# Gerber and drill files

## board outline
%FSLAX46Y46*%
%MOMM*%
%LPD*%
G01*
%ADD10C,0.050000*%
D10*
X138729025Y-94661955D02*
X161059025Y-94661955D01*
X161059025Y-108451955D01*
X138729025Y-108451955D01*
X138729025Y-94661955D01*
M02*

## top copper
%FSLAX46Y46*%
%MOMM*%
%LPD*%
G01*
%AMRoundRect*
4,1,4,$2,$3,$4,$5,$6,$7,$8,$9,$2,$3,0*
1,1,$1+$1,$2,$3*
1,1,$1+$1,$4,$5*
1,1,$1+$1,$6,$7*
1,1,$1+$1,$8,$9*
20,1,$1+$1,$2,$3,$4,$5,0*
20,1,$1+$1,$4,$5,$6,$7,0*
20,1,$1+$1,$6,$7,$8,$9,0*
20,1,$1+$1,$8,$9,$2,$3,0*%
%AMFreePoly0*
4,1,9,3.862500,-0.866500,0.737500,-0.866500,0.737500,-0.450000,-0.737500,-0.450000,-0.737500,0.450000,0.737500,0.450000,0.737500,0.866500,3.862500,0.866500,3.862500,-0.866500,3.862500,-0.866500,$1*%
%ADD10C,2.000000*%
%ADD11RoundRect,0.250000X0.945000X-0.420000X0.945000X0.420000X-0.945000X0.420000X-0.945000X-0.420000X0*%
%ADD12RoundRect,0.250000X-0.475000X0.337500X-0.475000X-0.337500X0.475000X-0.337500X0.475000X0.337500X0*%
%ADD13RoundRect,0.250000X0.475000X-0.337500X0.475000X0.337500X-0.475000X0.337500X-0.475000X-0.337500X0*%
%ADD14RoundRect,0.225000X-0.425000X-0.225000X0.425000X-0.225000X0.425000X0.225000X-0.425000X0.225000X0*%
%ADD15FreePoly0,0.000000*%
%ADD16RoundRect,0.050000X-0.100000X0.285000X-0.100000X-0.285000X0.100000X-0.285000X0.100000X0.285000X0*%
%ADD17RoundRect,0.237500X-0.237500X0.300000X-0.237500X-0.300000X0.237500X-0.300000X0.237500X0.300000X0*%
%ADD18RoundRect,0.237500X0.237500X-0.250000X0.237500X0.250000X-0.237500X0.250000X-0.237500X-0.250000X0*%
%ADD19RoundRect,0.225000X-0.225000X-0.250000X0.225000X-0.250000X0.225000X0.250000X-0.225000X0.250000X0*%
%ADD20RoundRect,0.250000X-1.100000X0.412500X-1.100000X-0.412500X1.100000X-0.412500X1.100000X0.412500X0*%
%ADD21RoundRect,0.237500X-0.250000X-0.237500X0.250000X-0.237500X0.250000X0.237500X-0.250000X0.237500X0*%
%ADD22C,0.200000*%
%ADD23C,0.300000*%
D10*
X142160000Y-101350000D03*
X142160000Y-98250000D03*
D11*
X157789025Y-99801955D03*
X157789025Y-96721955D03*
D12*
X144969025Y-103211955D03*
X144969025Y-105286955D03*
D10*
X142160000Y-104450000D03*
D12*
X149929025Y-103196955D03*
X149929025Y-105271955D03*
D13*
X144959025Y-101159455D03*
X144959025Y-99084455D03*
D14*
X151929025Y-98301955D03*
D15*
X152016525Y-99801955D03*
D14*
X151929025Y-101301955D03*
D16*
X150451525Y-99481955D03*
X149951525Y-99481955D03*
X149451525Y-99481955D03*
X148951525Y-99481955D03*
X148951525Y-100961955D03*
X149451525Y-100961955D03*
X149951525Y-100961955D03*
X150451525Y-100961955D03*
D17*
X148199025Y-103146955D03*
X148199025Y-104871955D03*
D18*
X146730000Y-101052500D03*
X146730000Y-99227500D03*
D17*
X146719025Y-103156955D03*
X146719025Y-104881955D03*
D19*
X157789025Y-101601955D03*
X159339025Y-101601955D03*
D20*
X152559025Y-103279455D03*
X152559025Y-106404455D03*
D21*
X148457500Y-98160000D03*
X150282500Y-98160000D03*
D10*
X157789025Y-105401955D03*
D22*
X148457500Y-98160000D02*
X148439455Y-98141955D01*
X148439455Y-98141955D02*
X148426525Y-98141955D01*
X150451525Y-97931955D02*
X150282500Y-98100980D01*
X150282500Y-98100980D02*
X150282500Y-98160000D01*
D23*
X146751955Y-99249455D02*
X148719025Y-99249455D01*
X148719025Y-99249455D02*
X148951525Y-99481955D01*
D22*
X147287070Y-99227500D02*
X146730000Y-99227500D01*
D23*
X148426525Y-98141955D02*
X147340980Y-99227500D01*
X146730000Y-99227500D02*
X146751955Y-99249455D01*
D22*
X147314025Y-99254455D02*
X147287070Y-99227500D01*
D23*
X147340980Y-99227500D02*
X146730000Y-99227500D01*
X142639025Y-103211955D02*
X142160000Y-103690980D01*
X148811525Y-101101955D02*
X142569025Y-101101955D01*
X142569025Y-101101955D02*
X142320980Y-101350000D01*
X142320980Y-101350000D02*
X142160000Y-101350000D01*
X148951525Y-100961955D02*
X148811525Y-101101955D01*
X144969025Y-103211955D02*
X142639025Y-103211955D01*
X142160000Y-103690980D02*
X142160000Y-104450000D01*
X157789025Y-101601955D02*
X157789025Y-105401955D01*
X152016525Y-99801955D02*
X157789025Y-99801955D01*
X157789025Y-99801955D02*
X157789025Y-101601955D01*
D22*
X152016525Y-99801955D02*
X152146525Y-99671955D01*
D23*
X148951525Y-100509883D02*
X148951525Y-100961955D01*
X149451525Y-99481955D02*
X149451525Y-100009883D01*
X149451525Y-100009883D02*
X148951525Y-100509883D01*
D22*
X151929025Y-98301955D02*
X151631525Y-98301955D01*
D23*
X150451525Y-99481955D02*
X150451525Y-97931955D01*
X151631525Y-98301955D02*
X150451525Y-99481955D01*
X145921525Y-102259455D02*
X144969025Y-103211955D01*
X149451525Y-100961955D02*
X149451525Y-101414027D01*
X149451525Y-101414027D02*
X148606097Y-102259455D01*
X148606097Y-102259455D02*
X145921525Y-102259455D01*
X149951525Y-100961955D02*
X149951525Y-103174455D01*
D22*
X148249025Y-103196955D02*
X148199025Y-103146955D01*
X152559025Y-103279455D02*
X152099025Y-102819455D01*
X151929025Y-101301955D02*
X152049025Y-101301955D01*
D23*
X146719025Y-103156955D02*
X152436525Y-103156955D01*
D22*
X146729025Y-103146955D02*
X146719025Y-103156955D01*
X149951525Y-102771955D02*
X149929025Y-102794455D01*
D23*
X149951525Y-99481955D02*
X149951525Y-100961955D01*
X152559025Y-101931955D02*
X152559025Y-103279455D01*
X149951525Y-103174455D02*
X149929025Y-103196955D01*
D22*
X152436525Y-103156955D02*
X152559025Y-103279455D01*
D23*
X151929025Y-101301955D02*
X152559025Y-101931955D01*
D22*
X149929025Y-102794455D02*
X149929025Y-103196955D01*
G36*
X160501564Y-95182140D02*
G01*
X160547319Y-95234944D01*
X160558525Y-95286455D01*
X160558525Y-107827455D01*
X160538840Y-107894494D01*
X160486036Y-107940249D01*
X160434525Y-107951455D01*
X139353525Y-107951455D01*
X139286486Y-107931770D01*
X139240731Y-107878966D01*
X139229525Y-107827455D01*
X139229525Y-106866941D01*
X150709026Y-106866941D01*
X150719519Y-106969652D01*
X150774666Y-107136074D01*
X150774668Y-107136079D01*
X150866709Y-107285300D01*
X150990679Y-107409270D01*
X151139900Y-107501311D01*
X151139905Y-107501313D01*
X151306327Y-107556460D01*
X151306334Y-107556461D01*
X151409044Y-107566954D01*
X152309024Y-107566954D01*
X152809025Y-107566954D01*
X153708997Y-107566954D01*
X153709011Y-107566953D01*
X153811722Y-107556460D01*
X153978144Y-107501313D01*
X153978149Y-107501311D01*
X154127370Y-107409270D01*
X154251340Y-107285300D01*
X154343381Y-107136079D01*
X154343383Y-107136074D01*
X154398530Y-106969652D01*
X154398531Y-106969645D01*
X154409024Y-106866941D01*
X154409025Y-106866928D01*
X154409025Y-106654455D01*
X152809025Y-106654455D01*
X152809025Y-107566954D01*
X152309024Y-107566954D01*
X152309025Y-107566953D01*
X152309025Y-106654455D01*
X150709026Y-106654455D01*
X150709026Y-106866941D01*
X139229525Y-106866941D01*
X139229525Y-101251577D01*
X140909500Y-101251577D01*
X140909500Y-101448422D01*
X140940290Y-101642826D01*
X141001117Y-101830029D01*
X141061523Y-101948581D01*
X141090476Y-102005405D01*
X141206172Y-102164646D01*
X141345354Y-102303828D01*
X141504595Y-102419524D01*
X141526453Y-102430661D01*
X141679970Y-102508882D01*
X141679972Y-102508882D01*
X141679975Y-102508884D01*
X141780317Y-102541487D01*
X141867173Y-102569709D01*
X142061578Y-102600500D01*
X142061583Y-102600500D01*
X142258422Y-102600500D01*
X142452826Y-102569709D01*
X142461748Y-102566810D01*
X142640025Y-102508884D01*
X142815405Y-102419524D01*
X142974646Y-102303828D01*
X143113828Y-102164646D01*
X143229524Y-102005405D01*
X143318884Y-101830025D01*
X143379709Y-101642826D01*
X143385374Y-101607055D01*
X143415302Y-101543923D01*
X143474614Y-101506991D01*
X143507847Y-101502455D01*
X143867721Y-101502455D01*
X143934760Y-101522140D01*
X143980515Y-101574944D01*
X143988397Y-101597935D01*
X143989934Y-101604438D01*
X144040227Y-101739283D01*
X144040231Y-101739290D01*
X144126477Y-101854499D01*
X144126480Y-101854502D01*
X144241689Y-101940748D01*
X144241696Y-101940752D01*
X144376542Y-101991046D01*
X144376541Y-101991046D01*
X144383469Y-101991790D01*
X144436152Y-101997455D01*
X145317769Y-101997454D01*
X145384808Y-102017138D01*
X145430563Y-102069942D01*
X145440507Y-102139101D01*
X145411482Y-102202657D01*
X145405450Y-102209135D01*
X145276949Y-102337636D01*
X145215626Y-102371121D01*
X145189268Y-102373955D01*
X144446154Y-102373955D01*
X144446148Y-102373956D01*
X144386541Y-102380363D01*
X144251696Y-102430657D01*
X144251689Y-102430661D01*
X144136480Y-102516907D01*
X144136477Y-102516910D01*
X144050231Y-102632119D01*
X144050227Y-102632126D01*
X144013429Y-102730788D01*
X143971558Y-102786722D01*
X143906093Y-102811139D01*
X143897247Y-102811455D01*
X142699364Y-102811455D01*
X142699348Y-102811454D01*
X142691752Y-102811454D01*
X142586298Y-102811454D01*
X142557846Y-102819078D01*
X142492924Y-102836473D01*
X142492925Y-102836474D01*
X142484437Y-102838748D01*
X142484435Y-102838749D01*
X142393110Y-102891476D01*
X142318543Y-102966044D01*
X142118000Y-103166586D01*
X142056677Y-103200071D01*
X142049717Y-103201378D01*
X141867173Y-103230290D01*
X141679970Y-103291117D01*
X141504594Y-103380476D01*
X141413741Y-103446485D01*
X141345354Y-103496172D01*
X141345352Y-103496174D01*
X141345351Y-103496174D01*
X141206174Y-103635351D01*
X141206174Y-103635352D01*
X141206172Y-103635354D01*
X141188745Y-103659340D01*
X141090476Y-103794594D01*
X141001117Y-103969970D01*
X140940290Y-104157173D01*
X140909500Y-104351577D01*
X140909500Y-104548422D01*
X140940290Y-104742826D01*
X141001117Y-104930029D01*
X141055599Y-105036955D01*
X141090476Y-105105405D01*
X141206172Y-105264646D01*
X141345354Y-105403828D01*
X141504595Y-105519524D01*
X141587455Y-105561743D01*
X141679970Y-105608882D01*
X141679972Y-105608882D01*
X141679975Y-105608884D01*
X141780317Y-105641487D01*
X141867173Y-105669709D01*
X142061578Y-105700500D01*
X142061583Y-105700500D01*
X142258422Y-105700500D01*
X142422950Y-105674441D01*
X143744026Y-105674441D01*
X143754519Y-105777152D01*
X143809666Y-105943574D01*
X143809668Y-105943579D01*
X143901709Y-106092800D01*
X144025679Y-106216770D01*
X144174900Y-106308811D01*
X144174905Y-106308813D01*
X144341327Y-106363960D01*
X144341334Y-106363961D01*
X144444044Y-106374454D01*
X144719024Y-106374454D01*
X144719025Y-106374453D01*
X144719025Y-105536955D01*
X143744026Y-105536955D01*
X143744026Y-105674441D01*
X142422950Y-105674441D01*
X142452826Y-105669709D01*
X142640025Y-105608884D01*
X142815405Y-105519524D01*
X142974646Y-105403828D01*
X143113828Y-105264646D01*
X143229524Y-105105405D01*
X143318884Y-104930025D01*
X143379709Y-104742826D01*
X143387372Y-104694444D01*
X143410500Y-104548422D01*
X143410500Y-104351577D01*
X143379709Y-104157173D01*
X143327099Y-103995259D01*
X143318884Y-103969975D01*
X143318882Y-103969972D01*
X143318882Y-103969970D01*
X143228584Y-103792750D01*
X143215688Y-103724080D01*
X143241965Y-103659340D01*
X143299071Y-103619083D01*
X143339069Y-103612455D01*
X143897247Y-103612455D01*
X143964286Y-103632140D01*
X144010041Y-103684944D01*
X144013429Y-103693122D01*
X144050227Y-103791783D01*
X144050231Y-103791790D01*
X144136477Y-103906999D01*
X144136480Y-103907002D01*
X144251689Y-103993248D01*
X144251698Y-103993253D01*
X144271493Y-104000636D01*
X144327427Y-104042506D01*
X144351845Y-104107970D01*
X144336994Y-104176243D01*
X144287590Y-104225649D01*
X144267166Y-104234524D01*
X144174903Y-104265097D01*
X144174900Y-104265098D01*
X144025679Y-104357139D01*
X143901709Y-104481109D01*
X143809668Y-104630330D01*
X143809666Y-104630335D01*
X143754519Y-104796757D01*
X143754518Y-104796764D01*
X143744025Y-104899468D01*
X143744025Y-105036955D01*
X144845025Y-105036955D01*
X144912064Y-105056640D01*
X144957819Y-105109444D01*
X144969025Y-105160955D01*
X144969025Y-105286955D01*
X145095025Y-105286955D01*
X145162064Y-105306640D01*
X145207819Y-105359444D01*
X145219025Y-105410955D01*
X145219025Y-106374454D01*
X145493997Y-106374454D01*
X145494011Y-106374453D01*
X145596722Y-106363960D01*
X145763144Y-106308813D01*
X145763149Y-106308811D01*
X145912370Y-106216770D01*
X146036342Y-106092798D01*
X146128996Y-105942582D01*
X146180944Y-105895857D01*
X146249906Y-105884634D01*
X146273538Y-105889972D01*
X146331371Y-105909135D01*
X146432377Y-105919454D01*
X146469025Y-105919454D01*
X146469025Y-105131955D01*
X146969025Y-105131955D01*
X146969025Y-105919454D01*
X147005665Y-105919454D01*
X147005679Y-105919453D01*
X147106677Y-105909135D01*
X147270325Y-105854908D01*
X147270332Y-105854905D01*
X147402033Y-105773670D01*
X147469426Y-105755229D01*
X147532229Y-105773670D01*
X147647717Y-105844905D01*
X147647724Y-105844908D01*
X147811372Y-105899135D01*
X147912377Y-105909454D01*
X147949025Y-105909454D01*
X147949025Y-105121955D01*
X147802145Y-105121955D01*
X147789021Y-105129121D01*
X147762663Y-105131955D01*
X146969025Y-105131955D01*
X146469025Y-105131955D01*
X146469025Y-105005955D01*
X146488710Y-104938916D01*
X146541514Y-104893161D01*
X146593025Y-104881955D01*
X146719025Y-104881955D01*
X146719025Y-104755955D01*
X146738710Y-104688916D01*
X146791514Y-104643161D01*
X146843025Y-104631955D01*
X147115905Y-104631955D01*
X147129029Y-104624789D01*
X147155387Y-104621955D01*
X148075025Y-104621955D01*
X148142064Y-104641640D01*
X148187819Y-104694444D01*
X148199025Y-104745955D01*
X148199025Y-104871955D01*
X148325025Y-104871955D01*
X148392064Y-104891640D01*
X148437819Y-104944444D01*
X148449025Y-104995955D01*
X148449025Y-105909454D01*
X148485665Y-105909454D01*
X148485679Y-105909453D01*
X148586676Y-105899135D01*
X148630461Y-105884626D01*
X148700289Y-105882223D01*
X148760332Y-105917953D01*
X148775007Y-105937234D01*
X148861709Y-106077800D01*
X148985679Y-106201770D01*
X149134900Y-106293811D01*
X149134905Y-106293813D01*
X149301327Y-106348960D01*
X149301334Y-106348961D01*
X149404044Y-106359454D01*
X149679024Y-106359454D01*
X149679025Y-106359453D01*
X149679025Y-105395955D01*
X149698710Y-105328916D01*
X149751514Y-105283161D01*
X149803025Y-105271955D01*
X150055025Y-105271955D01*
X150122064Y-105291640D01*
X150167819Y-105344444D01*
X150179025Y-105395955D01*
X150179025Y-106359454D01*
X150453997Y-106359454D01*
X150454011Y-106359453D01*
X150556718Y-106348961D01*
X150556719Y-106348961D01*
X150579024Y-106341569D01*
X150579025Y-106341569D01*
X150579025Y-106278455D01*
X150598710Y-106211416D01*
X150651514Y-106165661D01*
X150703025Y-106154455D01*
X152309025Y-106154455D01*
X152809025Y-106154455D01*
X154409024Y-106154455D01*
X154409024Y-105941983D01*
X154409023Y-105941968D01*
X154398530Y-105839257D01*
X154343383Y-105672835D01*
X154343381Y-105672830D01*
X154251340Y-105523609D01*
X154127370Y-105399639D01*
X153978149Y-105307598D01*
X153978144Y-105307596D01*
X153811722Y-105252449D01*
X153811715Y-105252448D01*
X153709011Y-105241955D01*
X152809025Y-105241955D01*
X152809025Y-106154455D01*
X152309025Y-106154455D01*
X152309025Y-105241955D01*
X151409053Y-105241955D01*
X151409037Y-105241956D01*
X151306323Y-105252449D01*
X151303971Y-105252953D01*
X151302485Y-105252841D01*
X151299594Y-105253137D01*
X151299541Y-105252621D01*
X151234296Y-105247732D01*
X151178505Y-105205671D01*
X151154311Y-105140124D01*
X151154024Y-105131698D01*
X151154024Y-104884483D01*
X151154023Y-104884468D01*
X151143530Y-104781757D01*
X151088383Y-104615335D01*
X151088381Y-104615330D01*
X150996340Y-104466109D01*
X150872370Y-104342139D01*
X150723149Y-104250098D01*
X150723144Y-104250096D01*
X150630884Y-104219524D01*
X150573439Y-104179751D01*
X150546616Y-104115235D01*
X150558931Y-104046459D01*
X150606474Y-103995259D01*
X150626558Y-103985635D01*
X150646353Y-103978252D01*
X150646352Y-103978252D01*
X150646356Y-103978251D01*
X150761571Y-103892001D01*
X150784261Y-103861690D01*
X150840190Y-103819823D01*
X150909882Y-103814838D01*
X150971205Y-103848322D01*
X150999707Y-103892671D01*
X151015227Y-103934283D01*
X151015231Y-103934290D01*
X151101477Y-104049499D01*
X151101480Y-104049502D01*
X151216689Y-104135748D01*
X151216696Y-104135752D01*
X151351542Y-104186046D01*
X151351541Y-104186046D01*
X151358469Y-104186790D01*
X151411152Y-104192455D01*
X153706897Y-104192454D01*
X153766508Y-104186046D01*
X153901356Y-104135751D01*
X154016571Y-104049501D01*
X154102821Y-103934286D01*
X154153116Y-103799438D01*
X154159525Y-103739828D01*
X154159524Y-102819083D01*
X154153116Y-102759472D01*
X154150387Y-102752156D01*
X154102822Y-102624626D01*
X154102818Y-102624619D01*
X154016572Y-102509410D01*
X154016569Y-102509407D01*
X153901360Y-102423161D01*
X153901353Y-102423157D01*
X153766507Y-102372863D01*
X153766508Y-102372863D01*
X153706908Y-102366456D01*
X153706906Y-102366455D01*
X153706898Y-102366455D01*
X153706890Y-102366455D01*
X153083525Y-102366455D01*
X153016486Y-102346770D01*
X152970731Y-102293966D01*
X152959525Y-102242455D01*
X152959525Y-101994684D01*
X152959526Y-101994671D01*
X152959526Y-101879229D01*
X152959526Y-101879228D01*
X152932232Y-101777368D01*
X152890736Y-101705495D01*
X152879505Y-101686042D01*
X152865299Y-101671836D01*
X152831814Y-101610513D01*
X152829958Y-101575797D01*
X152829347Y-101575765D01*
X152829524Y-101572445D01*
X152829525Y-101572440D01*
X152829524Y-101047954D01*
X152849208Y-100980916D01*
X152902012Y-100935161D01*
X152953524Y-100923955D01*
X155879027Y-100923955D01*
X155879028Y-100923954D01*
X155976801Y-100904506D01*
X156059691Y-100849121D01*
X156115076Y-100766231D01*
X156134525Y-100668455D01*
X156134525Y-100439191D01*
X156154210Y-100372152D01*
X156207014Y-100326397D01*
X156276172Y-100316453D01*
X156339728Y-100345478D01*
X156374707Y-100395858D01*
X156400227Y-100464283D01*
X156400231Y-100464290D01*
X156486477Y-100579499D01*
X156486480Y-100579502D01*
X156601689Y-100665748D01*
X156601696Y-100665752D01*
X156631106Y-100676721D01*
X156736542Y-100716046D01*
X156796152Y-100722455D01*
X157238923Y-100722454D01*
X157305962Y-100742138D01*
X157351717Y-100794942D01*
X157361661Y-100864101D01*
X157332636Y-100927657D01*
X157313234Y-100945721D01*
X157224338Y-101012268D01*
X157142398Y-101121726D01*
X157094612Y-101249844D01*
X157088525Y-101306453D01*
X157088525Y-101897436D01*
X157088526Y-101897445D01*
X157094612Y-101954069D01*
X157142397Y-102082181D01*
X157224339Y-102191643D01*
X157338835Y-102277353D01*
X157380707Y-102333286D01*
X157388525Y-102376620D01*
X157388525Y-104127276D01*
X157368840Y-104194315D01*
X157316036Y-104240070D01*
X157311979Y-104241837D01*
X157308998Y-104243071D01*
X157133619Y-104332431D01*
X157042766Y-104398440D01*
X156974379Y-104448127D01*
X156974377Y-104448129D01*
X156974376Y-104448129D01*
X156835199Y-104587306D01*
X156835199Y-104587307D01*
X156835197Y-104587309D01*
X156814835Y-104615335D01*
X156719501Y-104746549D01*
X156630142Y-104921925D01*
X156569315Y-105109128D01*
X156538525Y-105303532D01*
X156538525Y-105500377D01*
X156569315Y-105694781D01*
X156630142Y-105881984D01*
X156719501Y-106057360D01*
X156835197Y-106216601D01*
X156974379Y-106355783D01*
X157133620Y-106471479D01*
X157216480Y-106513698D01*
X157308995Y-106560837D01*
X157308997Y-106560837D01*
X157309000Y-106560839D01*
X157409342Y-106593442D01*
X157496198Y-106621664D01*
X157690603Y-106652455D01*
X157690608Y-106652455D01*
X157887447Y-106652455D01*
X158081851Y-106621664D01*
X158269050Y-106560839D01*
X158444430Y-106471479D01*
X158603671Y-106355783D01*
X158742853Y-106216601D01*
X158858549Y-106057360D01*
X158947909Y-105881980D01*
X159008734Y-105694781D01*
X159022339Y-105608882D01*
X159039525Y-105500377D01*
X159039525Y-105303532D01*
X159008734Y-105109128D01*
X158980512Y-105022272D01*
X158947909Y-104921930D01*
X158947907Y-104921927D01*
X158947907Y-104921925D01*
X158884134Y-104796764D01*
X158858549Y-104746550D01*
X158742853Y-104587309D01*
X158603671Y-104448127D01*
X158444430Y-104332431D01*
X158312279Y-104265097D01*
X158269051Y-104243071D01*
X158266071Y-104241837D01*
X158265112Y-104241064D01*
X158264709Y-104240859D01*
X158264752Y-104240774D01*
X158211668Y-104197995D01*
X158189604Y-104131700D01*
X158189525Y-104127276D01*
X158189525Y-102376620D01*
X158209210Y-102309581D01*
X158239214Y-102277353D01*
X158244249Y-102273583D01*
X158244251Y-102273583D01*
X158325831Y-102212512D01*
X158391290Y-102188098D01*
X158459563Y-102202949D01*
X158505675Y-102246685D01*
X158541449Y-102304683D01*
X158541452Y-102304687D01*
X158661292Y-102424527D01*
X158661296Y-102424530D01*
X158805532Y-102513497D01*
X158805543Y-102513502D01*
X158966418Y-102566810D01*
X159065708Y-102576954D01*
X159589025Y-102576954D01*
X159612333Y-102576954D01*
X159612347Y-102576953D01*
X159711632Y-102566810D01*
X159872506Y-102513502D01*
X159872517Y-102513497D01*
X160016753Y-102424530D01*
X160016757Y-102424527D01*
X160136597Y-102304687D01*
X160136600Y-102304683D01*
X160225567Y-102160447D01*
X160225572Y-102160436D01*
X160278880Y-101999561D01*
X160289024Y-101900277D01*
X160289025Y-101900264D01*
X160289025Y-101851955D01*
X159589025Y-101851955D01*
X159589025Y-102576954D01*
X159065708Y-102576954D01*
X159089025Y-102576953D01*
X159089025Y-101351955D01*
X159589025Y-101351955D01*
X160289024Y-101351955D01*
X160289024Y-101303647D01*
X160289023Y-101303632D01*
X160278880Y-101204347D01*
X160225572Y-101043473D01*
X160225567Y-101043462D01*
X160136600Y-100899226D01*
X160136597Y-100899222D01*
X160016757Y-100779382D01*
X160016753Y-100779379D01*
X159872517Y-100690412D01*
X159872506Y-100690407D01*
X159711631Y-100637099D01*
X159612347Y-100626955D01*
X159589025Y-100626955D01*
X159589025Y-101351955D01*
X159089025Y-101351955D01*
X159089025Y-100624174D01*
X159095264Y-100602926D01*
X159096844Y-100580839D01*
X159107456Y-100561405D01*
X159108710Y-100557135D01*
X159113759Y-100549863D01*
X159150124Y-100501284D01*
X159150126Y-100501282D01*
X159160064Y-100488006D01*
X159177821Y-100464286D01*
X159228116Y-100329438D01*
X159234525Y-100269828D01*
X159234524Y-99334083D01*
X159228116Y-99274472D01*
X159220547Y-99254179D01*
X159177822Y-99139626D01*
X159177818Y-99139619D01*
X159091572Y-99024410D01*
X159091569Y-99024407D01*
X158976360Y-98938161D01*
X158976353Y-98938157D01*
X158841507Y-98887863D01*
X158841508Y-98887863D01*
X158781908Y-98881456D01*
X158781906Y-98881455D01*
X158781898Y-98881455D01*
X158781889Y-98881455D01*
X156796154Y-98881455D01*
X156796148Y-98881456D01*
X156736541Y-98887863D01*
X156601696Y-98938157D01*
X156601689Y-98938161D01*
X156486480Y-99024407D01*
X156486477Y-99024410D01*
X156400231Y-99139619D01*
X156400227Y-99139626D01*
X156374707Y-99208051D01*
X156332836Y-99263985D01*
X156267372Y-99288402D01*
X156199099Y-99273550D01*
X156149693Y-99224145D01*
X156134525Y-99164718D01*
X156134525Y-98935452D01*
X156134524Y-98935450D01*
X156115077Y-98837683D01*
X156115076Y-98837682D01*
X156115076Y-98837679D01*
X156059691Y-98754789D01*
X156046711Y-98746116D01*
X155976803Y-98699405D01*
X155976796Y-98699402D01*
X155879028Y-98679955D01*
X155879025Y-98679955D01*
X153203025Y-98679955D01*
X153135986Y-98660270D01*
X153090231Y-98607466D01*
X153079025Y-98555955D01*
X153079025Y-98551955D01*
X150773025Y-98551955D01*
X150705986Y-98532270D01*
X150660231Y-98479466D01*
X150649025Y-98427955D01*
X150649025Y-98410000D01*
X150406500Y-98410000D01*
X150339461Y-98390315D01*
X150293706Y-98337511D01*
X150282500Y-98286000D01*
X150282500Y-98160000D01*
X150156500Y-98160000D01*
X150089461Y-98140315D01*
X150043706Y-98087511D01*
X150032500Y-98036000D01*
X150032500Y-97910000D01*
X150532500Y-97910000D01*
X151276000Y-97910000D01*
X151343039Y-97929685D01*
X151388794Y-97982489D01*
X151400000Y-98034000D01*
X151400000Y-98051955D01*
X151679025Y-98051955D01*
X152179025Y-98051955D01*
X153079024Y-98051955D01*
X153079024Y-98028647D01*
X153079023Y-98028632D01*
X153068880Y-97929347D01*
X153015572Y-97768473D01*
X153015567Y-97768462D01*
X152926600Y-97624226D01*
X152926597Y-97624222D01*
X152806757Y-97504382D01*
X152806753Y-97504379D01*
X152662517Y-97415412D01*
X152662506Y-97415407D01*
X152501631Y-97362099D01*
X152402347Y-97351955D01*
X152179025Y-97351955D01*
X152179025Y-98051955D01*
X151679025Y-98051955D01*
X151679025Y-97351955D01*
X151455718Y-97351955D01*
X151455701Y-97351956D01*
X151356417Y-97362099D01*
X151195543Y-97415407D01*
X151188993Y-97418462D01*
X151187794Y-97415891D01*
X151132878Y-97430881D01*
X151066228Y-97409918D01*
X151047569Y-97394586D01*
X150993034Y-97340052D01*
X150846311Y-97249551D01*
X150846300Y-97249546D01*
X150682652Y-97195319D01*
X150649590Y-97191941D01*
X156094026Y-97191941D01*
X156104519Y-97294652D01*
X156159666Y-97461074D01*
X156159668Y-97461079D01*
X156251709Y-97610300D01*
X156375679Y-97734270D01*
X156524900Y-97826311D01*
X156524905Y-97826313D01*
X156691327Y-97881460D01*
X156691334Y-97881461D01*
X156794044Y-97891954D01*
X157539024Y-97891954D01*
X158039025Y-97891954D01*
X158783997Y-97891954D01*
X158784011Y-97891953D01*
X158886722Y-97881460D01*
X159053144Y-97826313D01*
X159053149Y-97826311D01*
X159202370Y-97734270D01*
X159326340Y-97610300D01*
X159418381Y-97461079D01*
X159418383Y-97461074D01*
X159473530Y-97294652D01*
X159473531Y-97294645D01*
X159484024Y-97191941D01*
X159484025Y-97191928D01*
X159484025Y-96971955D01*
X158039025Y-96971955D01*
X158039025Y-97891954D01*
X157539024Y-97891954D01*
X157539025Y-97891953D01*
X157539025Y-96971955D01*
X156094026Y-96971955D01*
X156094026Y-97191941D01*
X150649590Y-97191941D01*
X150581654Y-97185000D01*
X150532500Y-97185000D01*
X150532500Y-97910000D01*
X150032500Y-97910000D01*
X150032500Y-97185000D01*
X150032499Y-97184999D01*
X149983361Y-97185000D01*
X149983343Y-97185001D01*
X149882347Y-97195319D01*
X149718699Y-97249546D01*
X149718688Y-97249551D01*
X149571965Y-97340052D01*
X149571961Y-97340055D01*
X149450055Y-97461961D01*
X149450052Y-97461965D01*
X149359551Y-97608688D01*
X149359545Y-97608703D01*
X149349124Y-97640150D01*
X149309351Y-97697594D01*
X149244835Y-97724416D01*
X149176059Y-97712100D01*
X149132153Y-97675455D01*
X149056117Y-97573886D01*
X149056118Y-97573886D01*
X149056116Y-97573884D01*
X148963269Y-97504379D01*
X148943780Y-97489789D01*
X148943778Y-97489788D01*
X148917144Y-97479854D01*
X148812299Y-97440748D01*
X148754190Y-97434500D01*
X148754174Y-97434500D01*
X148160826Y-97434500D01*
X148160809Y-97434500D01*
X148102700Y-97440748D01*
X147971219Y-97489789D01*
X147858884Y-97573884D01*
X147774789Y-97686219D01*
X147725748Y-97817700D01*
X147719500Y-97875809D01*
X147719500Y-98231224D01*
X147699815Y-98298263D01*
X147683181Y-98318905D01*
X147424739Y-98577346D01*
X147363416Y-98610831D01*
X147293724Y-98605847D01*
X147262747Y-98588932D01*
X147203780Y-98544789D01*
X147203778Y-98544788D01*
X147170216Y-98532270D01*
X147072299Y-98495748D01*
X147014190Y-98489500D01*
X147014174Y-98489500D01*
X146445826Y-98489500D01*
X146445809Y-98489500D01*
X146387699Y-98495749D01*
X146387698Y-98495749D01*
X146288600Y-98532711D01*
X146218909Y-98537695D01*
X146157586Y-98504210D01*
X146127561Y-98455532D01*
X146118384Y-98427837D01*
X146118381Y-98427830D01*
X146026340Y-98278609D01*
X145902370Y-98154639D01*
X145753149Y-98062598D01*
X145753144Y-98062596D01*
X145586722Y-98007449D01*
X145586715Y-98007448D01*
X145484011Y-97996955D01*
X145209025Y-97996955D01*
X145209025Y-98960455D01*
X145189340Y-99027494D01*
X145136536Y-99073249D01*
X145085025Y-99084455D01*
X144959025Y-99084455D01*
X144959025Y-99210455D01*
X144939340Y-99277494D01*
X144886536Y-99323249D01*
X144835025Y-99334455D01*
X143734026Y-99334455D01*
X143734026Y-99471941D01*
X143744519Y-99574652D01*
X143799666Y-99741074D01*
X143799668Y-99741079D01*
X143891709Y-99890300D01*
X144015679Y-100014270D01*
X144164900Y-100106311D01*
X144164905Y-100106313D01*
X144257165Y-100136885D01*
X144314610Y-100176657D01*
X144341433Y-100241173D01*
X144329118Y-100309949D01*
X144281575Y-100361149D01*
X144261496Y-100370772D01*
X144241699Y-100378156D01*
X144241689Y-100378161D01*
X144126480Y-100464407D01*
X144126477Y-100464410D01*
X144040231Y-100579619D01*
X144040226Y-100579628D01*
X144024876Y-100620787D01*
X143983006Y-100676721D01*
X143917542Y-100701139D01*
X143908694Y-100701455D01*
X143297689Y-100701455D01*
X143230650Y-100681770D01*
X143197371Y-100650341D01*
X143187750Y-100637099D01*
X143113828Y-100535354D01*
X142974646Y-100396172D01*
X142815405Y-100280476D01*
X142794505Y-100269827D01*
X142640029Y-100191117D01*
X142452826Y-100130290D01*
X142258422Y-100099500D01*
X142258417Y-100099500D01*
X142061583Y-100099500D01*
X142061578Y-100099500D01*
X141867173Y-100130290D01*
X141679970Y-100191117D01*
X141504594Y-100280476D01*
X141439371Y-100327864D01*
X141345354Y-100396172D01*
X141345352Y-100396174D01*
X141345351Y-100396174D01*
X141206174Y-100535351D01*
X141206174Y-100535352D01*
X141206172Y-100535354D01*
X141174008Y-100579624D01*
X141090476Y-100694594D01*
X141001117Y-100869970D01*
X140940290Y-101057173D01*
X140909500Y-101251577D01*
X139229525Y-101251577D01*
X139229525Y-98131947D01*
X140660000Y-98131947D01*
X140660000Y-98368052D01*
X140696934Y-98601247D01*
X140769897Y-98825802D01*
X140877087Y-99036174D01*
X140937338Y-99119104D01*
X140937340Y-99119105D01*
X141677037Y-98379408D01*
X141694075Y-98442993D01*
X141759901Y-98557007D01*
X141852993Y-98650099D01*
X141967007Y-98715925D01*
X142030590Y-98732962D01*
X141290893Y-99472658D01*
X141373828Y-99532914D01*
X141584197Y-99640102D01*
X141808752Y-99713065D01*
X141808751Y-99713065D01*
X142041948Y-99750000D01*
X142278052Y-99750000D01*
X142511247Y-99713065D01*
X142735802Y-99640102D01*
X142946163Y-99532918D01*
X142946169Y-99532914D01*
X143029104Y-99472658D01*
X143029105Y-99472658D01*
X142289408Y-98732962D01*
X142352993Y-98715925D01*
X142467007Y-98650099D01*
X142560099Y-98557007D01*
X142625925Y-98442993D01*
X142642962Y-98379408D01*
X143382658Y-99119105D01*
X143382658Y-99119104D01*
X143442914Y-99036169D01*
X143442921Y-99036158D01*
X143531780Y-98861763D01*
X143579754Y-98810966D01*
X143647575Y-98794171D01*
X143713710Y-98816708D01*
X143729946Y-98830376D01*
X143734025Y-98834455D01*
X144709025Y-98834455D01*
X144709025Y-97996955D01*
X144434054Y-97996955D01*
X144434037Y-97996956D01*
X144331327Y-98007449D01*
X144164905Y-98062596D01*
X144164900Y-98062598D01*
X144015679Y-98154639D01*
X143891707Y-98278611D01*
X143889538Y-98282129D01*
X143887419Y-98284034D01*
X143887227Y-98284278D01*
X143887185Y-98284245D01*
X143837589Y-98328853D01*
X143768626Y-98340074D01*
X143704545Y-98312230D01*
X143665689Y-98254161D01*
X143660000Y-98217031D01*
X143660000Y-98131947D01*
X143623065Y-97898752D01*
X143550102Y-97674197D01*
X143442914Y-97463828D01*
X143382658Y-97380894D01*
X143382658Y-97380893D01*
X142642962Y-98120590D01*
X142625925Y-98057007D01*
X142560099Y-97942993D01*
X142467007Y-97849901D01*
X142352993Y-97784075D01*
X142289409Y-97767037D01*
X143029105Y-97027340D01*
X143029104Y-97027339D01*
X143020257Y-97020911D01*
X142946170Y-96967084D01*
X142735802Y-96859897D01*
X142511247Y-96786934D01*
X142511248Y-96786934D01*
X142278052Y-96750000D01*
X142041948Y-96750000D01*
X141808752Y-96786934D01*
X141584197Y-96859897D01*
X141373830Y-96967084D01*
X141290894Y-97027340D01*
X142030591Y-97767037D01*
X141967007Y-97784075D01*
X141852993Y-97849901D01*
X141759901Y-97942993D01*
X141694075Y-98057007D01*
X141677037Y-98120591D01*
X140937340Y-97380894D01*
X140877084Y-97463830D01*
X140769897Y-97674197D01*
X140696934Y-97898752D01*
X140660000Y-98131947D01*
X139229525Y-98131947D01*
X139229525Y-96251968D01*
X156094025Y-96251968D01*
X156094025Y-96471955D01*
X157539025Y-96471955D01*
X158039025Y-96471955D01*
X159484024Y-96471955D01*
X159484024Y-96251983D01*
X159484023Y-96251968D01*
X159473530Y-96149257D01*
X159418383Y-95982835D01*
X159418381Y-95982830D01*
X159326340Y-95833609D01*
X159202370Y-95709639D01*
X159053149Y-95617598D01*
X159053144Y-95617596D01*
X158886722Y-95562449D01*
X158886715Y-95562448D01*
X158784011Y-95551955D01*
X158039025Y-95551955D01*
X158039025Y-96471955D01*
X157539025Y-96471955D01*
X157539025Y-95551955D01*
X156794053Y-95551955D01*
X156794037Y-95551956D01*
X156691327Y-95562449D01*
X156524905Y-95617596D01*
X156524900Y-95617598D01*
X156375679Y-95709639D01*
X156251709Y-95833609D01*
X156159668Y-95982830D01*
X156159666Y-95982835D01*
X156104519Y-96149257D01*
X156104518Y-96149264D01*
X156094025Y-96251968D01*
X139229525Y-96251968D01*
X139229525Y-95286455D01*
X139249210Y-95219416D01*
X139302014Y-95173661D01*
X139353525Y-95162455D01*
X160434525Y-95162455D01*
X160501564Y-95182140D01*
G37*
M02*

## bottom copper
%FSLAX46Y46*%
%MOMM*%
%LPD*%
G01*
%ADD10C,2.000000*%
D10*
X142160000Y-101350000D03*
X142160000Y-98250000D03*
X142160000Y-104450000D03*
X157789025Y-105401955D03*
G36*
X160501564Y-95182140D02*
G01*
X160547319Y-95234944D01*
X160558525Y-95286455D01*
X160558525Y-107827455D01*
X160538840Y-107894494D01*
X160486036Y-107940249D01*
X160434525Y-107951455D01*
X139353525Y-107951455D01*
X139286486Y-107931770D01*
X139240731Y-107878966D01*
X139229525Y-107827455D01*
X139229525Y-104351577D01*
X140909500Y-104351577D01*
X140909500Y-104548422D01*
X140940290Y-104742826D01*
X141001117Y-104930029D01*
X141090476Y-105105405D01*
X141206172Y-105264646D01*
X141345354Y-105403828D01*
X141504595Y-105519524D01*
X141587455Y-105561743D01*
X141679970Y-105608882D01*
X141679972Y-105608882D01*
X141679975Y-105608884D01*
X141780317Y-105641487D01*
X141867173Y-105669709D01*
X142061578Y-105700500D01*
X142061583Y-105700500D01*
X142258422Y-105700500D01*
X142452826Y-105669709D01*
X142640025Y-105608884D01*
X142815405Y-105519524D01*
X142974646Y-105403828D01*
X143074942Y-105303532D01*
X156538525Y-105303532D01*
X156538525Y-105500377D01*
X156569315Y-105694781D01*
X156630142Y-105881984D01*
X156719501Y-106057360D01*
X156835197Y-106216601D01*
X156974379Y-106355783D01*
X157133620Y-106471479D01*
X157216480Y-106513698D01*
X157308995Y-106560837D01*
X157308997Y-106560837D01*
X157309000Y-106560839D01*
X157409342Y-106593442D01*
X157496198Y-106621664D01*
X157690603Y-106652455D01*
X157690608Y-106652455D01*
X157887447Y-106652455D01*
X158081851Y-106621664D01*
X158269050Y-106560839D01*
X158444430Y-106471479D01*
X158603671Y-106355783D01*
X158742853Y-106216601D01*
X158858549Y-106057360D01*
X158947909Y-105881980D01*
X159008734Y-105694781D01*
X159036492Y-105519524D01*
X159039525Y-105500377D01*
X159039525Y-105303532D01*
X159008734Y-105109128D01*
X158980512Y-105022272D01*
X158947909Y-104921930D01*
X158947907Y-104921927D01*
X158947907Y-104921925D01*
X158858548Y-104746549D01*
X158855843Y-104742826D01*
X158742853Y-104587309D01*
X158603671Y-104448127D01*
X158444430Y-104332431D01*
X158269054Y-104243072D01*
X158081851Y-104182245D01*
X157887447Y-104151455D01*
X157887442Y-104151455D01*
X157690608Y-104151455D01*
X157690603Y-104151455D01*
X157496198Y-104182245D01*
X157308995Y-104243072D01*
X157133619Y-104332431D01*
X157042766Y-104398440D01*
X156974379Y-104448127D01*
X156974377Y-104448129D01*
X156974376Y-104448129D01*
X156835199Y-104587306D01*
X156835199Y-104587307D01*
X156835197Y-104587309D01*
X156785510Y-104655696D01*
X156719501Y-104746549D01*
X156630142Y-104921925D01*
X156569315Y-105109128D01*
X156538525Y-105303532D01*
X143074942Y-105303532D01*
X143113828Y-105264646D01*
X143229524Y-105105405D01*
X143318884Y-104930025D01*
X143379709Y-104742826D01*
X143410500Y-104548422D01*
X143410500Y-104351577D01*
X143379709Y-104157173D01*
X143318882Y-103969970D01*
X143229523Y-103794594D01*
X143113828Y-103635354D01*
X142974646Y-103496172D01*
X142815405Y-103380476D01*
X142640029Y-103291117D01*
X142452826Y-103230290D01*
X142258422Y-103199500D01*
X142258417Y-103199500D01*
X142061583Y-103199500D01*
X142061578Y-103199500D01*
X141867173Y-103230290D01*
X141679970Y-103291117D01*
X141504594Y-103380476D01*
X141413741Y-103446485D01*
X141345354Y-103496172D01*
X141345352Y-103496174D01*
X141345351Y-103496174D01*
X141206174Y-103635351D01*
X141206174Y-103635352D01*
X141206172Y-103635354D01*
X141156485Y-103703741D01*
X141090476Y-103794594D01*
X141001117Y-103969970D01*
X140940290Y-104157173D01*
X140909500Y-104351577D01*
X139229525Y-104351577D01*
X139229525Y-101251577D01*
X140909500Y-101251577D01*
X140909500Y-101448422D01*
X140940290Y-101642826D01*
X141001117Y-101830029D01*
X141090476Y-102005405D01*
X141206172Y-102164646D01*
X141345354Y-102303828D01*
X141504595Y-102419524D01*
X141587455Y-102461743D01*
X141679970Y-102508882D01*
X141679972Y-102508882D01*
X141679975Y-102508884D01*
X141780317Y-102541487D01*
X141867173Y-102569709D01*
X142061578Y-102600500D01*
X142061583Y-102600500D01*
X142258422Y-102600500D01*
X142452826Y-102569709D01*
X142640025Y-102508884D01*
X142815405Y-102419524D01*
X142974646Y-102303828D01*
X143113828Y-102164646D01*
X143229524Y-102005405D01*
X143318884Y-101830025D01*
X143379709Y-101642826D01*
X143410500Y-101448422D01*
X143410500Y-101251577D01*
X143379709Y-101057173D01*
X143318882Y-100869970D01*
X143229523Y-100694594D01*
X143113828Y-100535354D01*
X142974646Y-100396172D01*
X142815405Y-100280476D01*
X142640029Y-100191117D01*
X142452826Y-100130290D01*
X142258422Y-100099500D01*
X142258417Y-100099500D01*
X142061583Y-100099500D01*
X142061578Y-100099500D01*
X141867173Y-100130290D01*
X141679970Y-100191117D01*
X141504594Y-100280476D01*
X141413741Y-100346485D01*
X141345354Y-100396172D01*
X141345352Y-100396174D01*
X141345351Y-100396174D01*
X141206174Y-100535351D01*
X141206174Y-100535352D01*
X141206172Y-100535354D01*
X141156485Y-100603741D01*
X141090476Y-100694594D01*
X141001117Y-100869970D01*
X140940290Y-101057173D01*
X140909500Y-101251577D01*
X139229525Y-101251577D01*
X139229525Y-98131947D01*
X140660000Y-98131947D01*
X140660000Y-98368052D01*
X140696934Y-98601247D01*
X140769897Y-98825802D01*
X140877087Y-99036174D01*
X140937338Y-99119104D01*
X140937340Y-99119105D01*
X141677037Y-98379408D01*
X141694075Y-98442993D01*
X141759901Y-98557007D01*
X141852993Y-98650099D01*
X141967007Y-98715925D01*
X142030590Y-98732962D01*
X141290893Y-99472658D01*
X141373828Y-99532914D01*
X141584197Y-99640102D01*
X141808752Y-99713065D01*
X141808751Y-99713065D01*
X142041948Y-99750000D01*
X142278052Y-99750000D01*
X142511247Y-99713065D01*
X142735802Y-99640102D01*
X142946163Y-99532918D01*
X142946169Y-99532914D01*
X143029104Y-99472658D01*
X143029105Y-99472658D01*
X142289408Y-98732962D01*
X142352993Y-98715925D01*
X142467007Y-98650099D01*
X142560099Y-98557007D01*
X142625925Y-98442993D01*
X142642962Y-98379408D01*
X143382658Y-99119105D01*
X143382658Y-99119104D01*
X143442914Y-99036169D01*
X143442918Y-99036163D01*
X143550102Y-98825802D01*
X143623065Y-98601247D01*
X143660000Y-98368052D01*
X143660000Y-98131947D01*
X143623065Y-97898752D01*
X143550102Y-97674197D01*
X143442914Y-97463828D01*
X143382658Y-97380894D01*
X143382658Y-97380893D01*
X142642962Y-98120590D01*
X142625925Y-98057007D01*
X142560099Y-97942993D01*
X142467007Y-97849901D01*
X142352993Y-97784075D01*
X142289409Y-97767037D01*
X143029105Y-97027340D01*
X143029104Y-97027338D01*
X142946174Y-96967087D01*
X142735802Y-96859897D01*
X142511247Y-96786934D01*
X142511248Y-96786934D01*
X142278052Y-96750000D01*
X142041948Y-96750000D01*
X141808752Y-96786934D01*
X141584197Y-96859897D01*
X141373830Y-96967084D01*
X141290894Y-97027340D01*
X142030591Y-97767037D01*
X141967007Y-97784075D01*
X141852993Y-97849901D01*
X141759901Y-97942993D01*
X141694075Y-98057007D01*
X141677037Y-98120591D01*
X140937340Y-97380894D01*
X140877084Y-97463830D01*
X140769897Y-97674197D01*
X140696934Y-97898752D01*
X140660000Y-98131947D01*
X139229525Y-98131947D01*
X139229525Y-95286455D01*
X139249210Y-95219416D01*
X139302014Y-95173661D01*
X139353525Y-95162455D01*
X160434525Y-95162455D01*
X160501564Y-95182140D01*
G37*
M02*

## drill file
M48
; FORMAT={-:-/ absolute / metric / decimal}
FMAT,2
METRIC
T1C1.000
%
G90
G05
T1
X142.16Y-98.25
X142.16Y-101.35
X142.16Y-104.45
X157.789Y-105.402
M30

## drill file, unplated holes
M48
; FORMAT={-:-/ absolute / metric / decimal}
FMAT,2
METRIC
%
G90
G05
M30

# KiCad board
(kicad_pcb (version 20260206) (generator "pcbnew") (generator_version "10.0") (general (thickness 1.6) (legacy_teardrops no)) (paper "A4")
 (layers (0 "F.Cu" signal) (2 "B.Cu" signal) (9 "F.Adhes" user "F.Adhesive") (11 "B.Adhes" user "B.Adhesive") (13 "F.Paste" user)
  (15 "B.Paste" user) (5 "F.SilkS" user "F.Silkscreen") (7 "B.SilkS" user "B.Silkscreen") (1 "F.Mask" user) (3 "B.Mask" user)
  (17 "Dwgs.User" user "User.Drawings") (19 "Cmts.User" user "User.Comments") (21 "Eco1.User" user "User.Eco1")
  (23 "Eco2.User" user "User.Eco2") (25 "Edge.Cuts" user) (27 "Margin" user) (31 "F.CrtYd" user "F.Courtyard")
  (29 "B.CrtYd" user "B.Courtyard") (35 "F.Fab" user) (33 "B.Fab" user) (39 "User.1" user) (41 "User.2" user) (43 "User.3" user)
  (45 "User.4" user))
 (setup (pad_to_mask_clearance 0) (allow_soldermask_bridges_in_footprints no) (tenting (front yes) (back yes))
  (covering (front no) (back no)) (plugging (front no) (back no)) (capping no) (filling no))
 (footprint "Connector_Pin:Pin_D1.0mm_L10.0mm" (layer "F.Cu") (at 142.16 101.35)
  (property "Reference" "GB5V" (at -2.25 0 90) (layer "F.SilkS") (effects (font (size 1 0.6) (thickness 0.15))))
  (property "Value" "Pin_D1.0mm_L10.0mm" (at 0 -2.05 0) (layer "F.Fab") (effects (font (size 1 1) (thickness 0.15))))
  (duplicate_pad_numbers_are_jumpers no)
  (pad "1" thru_hole circle (at 0 0) (size 2 2) (drill 1) (layers "*.Cu" "*.Mask") (remove_unused_layers no) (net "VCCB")))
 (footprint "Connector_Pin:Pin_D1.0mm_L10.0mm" (layer "F.Cu") (at 142.16 98.25)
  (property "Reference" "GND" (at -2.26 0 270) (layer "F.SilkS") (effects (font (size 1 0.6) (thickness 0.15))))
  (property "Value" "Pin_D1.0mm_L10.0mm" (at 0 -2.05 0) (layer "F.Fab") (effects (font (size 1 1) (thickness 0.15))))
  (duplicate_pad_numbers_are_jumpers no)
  (pad "1" thru_hole circle (at 0 0) (size 2 2) (drill 1) (layers "*.Cu" "*.Mask") (remove_unused_layers no) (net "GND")))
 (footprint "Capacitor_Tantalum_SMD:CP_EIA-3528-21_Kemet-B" (layer "F.Cu") (at 157.789025 98.261955 90)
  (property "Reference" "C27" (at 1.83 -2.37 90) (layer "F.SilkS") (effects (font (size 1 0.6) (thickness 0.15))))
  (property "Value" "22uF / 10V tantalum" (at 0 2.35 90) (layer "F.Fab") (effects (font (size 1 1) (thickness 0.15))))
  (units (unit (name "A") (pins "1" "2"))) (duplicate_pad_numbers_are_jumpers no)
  (pad "1" smd roundrect (at -1.54 0 90) (size 1.34 2.39) (layers "F.Cu" "F.Mask" "F.Paste") (roundrect_rratio 0.186567) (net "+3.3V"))
  (pad "2" smd roundrect (at 1.54 0 90) (size 1.34 2.39) (layers "F.Cu" "F.Mask" "F.Paste") (roundrect_rratio 0.186567) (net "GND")))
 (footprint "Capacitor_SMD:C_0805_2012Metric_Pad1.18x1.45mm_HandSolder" (layer "F.Cu") (at 144.969025 104.249455 -90)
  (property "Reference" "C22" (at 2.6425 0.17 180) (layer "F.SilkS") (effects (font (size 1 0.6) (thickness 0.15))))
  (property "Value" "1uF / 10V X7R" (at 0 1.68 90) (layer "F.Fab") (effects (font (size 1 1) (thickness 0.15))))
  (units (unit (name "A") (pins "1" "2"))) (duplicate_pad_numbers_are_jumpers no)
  (pad "1" smd roundrect (at -1.0375 0 270) (size 1.175 1.45) (layers "F.Cu" "F.Mask" "F.Paste") (roundrect_rratio 0.212766)
   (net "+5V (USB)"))
  (pad "2" smd roundrect (at 1.0375 0 270) (size 1.175 1.45) (layers "F.Cu" "F.Mask" "F.Paste") (roundrect_rratio 0.212766) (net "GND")))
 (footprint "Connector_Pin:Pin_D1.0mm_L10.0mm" (layer "F.Cu") (at 142.16 104.45)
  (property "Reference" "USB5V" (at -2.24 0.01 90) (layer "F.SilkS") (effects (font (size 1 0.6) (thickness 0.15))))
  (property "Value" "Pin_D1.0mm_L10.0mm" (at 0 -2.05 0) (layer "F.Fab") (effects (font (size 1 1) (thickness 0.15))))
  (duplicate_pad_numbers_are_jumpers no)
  (pad "1" thru_hole circle (at 0 0) (size 2 2) (drill 1) (layers "*.Cu" "*.Mask") (remove_unused_layers no) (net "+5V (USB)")))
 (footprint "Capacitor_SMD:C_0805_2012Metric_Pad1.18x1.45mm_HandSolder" (layer "F.Cu") (at 149.929025 104.234455 -90)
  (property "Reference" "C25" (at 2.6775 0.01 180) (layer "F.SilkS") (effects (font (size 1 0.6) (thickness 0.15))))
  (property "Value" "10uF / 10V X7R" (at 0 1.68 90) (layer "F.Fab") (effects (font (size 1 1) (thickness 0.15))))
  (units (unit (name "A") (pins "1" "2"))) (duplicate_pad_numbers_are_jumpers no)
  (pad "1" smd roundrect (at -1.0375 0 270) (size 1.175 1.45) (layers "F.Cu" "F.Mask" "F.Paste") (roundrect_rratio 0.212766)
   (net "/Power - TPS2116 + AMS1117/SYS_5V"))
  (pad "2" smd roundrect (at 1.0375 0 270) (size 1.175 1.45) (layers "F.Cu" "F.Mask" "F.Paste") (roundrect_rratio 0.212766) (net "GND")))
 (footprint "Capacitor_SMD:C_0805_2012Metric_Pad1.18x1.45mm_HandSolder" (layer "F.Cu") (at 144.959025 100.121955 90)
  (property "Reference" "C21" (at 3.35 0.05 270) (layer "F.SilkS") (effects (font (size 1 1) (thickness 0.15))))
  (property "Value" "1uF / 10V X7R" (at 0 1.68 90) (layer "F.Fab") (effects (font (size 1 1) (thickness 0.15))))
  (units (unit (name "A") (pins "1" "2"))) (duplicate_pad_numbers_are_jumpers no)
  (pad "1" smd roundrect (at -1.0375 0 90) (size 1.175 1.45) (layers "F.Cu" "F.Mask" "F.Paste") (roundrect_rratio 0.212766) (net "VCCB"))
  (pad "2" smd roundrect (at 1.0375 0 90) (size 1.175 1.45) (layers "F.Cu" "F.Mask" "F.Paste") (roundrect_rratio 0.212766) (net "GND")))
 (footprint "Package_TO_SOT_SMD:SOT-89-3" (layer "F.Cu") (at 153.879025 99.801955)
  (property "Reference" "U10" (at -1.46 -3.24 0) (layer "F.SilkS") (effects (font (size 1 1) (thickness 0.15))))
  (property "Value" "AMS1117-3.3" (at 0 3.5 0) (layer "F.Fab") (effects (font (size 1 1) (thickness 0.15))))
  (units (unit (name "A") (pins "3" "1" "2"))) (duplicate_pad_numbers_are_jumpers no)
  (pad "1" smd roundrect (at -1.95 -1.5) (size 1.3 0.9) (layers "F.Cu" "F.Mask" "F.Paste") (roundrect_rratio 0.25) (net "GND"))
  (pad "2" smd custom (at -1.8625 0) (size 1.475 0.9) (layers "F.Cu" "F.Mask" "F.Paste") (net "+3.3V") (zone_connect 2)
   (thermal_bridge_angle 45) (options (clearance outline) (anchor rect)) (primitives))
  (pad "3" smd roundrect (at -1.95 1.5) (size 1.3 0.9) (layers "F.Cu" "F.Mask" "F.Paste") (roundrect_rratio 0.25)
   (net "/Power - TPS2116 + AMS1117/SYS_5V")))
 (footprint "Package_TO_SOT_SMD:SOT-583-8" (layer "F.Cu") (at 149.701525 100.221955 -90)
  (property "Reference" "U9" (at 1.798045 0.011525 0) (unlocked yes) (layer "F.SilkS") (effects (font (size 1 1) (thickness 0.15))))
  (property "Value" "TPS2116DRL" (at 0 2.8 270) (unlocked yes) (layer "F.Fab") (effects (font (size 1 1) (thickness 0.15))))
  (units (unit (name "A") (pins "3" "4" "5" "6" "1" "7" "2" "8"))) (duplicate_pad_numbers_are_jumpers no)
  (pad "1" smd roundrect (at -0.74 -0.75 270) (size 0.67 0.3) (layers "F.Cu" "F.Mask" "F.Paste") (roundrect_rratio 0.1666666667) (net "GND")
   (thermal_bridge_angle 45))
  (pad "2" smd roundrect (at -0.74 -0.25 270) (size 0.67 0.3) (layers "F.Cu" "F.Mask" "F.Paste") (roundrect_rratio 0.1666666667)
   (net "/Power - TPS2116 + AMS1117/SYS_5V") (thermal_bridge_angle 45))
  (pad "3" smd roundrect (at -0.74 0.25 270) (size 0.67 0.3) (layers "F.Cu" "F.Mask" "F.Paste") (roundrect_rratio 0.1666666667) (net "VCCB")
   (thermal_bridge_angle 45))
  (pad "4" smd roundrect (at -0.74 0.75 270) (size 0.67 0.3) (layers "F.Cu" "F.Mask" "F.Paste") (roundrect_rratio 0.1666666667)
   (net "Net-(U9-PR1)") (thermal_bridge_angle 45))
  (pad "5" smd roundrect (at 0.74 0.75 270) (size 0.67 0.3) (layers "F.Cu" "F.Mask" "F.Paste") (roundrect_rratio 0.1666666667) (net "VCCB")
   (thermal_bridge_angle 45))
  (pad "6" smd roundrect (at 0.74 0.25 270) (size 0.67 0.3) (layers "F.Cu" "F.Mask" "F.Paste") (roundrect_rratio 0.1666666667)
   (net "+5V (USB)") (thermal_bridge_angle 45))
  (pad "7" smd roundrect (at 0.74 -0.25 270) (size 0.67 0.3) (layers "F.Cu" "F.Mask" "F.Paste") (roundrect_rratio 0.1666666667)
   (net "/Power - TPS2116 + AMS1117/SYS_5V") (thermal_bridge_angle 45))
  (pad "8" smd roundrect (at 0.74 -0.75 270) (size 0.67 0.3) (layers "F.Cu" "F.Mask" "F.Paste") (roundrect_rratio 0.1666666667)
   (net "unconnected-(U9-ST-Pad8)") (thermal_bridge_angle 45)))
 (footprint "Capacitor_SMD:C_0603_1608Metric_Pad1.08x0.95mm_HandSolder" (layer "F.Cu") (at 148.199025 104.009455 -90)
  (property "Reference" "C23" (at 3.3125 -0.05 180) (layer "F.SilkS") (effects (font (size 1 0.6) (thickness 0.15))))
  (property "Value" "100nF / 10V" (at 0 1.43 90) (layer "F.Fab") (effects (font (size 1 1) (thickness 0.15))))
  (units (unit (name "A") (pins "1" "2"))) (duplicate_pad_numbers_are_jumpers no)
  (pad "1" smd roundrect (at -0.8625 0 270) (size 1.075 0.95) (layers "F.Cu" "F.Mask" "F.Paste") (roundrect_rratio 0.25)
   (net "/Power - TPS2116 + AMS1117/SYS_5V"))
  (pad "2" smd roundrect (at 0.8625 0 270) (size 1.075 0.95) (layers "F.Cu" "F.Mask" "F.Paste") (roundrect_rratio 0.25) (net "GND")))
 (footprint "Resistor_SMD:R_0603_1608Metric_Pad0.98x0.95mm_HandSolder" (layer "F.Cu") (at 146.73 100.14 90)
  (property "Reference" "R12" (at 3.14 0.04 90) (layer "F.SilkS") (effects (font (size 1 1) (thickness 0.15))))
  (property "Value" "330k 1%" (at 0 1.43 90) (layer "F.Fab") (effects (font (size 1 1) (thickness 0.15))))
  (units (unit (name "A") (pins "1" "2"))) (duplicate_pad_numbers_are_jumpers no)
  (pad "1" smd roundrect (at -0.9125 0 90) (size 0.975 0.95) (layers "F.Cu" "F.Mask" "F.Paste") (roundrect_rratio 0.25) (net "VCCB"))
  (pad "2" smd roundrect (at 0.9125 0 90) (size 0.975 0.95) (layers "F.Cu" "F.Mask" "F.Paste") (roundrect_rratio 0.25) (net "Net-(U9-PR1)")))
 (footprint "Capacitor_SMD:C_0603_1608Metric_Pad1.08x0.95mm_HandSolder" (layer "F.Cu") (at 146.719025 104.019455 -90)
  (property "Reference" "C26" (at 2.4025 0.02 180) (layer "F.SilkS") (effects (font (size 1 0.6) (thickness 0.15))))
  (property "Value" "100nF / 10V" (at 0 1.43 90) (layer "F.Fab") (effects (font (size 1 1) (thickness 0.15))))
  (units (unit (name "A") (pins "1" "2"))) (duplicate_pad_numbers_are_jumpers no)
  (pad "1" smd roundrect (at -0.8625 0 270) (size 1.075 0.95) (layers "F.Cu" "F.Mask" "F.Paste") (roundrect_rratio 0.25)
   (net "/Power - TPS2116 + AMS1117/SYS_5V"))
  (pad "2" smd roundrect (at 0.8625 0 270) (size 1.075 0.95) (layers "F.Cu" "F.Mask" "F.Paste") (roundrect_rratio 0.25) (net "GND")))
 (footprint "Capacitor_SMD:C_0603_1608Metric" (layer "F.Cu") (at 158.564025 101.601955)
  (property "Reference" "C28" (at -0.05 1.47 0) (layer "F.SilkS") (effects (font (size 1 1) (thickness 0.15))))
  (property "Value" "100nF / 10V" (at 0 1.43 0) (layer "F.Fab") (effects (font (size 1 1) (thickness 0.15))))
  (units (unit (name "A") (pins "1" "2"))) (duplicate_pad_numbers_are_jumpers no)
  (pad "1" smd roundrect (at -0.775 0) (size 0.9 0.95) (layers "F.Cu" "F.Mask" "F.Paste") (roundrect_rratio 0.25) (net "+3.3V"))
  (pad "2" smd roundrect (at 0.775 0) (size 0.9 0.95) (layers "F.Cu" "F.Mask" "F.Paste") (roundrect_rratio 0.25) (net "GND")))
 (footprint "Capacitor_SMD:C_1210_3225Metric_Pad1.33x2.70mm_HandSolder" (layer "F.Cu") (at 152.559025 104.841955 -90)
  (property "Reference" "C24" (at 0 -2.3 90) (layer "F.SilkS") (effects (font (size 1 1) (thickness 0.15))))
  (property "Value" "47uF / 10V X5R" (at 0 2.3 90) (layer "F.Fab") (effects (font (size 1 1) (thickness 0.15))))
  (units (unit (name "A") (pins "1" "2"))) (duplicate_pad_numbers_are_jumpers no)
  (pad "1" smd roundrect (at -1.5625 0 270) (size 1.325 2.7) (layers "F.Cu" "F.Mask" "F.Paste") (roundrect_rratio 0.188679)
   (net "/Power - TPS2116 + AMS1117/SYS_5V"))
  (pad "2" smd roundrect (at 1.5625 0 270) (size 1.325 2.7) (layers "F.Cu" "F.Mask" "F.Paste") (roundrect_rratio 0.188679) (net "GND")))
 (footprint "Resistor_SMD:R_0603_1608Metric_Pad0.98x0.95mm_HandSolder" (layer "F.Cu") (at 149.37 98.16)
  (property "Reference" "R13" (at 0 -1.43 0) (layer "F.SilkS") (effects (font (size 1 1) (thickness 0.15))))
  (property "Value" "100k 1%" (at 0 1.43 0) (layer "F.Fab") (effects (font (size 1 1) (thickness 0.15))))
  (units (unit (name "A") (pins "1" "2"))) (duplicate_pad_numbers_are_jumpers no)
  (pad "1" smd roundrect (at -0.9125 0) (size 0.975 0.95) (layers "F.Cu" "F.Mask" "F.Paste") (roundrect_rratio 0.25) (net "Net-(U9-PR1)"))
  (pad "2" smd roundrect (at 0.9125 0) (size 0.975 0.95) (layers "F.Cu" "F.Mask" "F.Paste") (roundrect_rratio 0.25) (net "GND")))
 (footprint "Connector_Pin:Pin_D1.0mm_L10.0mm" (layer "F.Cu") (at 157.789025 105.401955)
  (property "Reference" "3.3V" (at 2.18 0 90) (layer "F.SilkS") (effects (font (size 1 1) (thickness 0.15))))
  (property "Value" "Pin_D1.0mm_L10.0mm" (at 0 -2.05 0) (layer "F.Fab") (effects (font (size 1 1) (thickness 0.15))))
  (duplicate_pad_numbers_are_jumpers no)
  (pad "1" thru_hole circle (at 0 0) (size 2 2) (drill 1) (layers "*.Cu" "*.Mask") (remove_unused_layers no) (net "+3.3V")))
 (gr_rect (start 138.729025 94.661955) (end 161.059025 108.451955) (stroke (width 0.05) (type default)) (fill no) (layer "Edge.Cuts"))
 (segment (start 148.811525 101.101955) (end 142.569025 101.101955) (width 0.3) (layer "F.Cu") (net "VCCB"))
 (segment (start 142.569025 101.101955) (end 142.32098 101.35) (width 0.3) (layer "F.Cu") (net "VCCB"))
 (segment (start 142.32098 101.35) (end 142.16 101.35) (width 0.3) (layer "F.Cu") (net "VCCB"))
 (segment (start 148.951525 100.509883) (end 148.951525 100.961955) (width 0.3) (layer "F.Cu") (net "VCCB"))
 (segment (start 149.451525 99.481955) (end 149.451525 100.009883) (width 0.3) (layer "F.Cu") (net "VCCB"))
 (segment (start 148.951525 100.961955) (end 148.811525 101.101955) (width 0.3) (layer "F.Cu") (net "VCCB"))
 (segment (start 149.451525 100.009883) (end 148.951525 100.509883) (width 0.3) (layer "F.Cu") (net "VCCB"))
 (segment (start 151.929025 98.301955) (end 151.631525 98.301955) (width 0.2) (layer "F.Cu") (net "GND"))
 (segment (start 150.451525 99.481955) (end 150.451525 97.931955) (width 0.3) (layer "F.Cu") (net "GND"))
 (segment (start 150.2825 98.10098) (end 150.2825 98.16) (width 0.2) (layer "F.Cu") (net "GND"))
 (segment (start 151.631525 98.301955) (end 150.451525 99.481955) (width 0.3) (layer "F.Cu") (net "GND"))
 (segment (start 150.451525 97.931955) (end 150.2825 98.10098) (width 0.2) (layer "F.Cu") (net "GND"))
 (segment (start 157.789025 101.601955) (end 157.789025 105.401955) (width 0.3) (layer "F.Cu") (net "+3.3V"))
 (segment (start 152.016525 99.801955) (end 157.789025 99.801955) (width 0.3) (layer "F.Cu") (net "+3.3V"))
 (segment (start 157.789025 99.801955) (end 157.789025 101.601955) (width 0.3) (layer "F.Cu") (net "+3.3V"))
 (segment (start 152.016525 99.801955) (end 152.146525 99.671955) (width 0.2) (layer "F.Cu") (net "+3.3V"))
 (segment (start 142.639025 103.211955) (end 142.16 103.69098) (width 0.3) (layer "F.Cu") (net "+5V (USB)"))
 (segment (start 145.921525 102.259455) (end 144.969025 103.211955) (width 0.3) (layer "F.Cu") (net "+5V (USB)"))
 (segment (start 142.16 103.69098) (end 142.16 104.45) (width 0.3) (layer "F.Cu") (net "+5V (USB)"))
 (segment (start 144.969025 103.211955) (end 142.639025 103.211955) (width 0.3) (layer "F.Cu") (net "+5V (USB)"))
 (segment (start 149.451525 100.961955) (end 149.451525 101.414027) (width 0.3) (layer "F.Cu") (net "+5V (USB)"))
 (segment (start 149.451525 101.414027) (end 148.606097 102.259455) (width 0.3) (layer "F.Cu") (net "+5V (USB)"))
 (segment (start 148.606097 102.259455) (end 145.921525 102.259455) (width 0.3) (layer "F.Cu") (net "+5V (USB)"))
 (segment (start 149.951525 100.961955) (end 149.951525 103.174455) (width 0.3) (layer "F.Cu") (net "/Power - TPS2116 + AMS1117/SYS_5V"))
 (segment (start 148.249025 103.196955) (end 148.199025 103.146955) (width 0.2) (layer "F.Cu") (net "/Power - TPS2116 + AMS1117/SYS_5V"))
 (segment (start 152.559025 103.279455) (end 152.099025 102.819455) (width 0.2) (layer "F.Cu") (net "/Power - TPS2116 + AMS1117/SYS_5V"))
 (segment (start 151.929025 101.301955) (end 152.049025 101.301955) (width 0.2) (layer "F.Cu") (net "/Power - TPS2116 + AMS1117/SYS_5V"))
 (segment (start 146.719025 103.156955) (end 152.436525 103.156955) (width 0.3) (layer "F.Cu") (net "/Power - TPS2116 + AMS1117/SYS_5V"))
 (segment (start 146.729025 103.146955) (end 146.719025 103.156955) (width 0.2) (layer "F.Cu") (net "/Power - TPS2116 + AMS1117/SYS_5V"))
 (segment (start 149.951525 102.771955) (end 149.929025 102.794455) (width 0.2) (layer "F.Cu") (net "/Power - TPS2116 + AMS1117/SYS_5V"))
 (segment (start 149.951525 99.481955) (end 149.951525 100.961955) (width 0.3) (layer "F.Cu") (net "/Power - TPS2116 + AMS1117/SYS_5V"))
 (segment (start 152.559025 101.931955) (end 152.559025 103.279455) (width 0.3) (layer "F.Cu") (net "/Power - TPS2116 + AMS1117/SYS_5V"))
 (segment (start 149.951525 103.174455) (end 149.929025 103.196955) (width 0.3) (layer "F.Cu") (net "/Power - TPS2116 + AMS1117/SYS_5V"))
 (segment (start 152.436525 103.156955) (end 152.559025 103.279455) (width 0.2) (layer "F.Cu") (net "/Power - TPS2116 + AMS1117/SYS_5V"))
 (segment (start 151.929025 101.301955) (end 152.559025 101.931955) (width 0.3) (layer "F.Cu") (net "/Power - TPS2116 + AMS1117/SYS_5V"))
 (segment (start 149.929025 102.794455) (end 149.929025 103.196955) (width 0.2) (layer "F.Cu") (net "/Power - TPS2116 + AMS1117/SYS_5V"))
 (segment (start 146.751955 99.249455) (end 148.719025 99.249455) (width 0.3) (layer "F.Cu") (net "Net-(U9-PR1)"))
 (segment (start 148.719025 99.249455) (end 148.951525 99.481955) (width 0.3) (layer "F.Cu") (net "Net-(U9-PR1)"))
 (segment (start 147.314025 99.254455) (end 147.28707 99.2275) (width 0.2) (layer "F.Cu") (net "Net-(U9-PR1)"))
 (segment (start 147.28707 99.2275) (end 146.73 99.2275) (width 0.2) (layer "F.Cu") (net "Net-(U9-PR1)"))
 (segment (start 146.73 99.2275) (end 146.751955 99.249455) (width 0.3) (layer "F.Cu") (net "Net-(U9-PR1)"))
 (segment (start 148.439455 98.141955) (end 148.426525 98.141955) (width 0.2) (layer "F.Cu") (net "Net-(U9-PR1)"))
 (segment (start 148.4575 98.16) (end 148.439455 98.141955) (width 0.2) (layer "F.Cu") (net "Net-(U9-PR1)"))
 (segment (start 148.426525 98.141955) (end 147.34098 99.2275) (width 0.3) (layer "F.Cu") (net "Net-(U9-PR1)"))
 (segment (start 147.34098 99.2275) (end 146.73 99.2275) (width 0.3) (layer "F.Cu") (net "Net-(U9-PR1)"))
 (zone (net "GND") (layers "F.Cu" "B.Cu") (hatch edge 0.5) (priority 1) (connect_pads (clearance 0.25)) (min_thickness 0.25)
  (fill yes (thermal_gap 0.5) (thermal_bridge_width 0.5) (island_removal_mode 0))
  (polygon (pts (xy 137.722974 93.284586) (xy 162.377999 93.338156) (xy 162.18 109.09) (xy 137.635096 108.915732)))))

